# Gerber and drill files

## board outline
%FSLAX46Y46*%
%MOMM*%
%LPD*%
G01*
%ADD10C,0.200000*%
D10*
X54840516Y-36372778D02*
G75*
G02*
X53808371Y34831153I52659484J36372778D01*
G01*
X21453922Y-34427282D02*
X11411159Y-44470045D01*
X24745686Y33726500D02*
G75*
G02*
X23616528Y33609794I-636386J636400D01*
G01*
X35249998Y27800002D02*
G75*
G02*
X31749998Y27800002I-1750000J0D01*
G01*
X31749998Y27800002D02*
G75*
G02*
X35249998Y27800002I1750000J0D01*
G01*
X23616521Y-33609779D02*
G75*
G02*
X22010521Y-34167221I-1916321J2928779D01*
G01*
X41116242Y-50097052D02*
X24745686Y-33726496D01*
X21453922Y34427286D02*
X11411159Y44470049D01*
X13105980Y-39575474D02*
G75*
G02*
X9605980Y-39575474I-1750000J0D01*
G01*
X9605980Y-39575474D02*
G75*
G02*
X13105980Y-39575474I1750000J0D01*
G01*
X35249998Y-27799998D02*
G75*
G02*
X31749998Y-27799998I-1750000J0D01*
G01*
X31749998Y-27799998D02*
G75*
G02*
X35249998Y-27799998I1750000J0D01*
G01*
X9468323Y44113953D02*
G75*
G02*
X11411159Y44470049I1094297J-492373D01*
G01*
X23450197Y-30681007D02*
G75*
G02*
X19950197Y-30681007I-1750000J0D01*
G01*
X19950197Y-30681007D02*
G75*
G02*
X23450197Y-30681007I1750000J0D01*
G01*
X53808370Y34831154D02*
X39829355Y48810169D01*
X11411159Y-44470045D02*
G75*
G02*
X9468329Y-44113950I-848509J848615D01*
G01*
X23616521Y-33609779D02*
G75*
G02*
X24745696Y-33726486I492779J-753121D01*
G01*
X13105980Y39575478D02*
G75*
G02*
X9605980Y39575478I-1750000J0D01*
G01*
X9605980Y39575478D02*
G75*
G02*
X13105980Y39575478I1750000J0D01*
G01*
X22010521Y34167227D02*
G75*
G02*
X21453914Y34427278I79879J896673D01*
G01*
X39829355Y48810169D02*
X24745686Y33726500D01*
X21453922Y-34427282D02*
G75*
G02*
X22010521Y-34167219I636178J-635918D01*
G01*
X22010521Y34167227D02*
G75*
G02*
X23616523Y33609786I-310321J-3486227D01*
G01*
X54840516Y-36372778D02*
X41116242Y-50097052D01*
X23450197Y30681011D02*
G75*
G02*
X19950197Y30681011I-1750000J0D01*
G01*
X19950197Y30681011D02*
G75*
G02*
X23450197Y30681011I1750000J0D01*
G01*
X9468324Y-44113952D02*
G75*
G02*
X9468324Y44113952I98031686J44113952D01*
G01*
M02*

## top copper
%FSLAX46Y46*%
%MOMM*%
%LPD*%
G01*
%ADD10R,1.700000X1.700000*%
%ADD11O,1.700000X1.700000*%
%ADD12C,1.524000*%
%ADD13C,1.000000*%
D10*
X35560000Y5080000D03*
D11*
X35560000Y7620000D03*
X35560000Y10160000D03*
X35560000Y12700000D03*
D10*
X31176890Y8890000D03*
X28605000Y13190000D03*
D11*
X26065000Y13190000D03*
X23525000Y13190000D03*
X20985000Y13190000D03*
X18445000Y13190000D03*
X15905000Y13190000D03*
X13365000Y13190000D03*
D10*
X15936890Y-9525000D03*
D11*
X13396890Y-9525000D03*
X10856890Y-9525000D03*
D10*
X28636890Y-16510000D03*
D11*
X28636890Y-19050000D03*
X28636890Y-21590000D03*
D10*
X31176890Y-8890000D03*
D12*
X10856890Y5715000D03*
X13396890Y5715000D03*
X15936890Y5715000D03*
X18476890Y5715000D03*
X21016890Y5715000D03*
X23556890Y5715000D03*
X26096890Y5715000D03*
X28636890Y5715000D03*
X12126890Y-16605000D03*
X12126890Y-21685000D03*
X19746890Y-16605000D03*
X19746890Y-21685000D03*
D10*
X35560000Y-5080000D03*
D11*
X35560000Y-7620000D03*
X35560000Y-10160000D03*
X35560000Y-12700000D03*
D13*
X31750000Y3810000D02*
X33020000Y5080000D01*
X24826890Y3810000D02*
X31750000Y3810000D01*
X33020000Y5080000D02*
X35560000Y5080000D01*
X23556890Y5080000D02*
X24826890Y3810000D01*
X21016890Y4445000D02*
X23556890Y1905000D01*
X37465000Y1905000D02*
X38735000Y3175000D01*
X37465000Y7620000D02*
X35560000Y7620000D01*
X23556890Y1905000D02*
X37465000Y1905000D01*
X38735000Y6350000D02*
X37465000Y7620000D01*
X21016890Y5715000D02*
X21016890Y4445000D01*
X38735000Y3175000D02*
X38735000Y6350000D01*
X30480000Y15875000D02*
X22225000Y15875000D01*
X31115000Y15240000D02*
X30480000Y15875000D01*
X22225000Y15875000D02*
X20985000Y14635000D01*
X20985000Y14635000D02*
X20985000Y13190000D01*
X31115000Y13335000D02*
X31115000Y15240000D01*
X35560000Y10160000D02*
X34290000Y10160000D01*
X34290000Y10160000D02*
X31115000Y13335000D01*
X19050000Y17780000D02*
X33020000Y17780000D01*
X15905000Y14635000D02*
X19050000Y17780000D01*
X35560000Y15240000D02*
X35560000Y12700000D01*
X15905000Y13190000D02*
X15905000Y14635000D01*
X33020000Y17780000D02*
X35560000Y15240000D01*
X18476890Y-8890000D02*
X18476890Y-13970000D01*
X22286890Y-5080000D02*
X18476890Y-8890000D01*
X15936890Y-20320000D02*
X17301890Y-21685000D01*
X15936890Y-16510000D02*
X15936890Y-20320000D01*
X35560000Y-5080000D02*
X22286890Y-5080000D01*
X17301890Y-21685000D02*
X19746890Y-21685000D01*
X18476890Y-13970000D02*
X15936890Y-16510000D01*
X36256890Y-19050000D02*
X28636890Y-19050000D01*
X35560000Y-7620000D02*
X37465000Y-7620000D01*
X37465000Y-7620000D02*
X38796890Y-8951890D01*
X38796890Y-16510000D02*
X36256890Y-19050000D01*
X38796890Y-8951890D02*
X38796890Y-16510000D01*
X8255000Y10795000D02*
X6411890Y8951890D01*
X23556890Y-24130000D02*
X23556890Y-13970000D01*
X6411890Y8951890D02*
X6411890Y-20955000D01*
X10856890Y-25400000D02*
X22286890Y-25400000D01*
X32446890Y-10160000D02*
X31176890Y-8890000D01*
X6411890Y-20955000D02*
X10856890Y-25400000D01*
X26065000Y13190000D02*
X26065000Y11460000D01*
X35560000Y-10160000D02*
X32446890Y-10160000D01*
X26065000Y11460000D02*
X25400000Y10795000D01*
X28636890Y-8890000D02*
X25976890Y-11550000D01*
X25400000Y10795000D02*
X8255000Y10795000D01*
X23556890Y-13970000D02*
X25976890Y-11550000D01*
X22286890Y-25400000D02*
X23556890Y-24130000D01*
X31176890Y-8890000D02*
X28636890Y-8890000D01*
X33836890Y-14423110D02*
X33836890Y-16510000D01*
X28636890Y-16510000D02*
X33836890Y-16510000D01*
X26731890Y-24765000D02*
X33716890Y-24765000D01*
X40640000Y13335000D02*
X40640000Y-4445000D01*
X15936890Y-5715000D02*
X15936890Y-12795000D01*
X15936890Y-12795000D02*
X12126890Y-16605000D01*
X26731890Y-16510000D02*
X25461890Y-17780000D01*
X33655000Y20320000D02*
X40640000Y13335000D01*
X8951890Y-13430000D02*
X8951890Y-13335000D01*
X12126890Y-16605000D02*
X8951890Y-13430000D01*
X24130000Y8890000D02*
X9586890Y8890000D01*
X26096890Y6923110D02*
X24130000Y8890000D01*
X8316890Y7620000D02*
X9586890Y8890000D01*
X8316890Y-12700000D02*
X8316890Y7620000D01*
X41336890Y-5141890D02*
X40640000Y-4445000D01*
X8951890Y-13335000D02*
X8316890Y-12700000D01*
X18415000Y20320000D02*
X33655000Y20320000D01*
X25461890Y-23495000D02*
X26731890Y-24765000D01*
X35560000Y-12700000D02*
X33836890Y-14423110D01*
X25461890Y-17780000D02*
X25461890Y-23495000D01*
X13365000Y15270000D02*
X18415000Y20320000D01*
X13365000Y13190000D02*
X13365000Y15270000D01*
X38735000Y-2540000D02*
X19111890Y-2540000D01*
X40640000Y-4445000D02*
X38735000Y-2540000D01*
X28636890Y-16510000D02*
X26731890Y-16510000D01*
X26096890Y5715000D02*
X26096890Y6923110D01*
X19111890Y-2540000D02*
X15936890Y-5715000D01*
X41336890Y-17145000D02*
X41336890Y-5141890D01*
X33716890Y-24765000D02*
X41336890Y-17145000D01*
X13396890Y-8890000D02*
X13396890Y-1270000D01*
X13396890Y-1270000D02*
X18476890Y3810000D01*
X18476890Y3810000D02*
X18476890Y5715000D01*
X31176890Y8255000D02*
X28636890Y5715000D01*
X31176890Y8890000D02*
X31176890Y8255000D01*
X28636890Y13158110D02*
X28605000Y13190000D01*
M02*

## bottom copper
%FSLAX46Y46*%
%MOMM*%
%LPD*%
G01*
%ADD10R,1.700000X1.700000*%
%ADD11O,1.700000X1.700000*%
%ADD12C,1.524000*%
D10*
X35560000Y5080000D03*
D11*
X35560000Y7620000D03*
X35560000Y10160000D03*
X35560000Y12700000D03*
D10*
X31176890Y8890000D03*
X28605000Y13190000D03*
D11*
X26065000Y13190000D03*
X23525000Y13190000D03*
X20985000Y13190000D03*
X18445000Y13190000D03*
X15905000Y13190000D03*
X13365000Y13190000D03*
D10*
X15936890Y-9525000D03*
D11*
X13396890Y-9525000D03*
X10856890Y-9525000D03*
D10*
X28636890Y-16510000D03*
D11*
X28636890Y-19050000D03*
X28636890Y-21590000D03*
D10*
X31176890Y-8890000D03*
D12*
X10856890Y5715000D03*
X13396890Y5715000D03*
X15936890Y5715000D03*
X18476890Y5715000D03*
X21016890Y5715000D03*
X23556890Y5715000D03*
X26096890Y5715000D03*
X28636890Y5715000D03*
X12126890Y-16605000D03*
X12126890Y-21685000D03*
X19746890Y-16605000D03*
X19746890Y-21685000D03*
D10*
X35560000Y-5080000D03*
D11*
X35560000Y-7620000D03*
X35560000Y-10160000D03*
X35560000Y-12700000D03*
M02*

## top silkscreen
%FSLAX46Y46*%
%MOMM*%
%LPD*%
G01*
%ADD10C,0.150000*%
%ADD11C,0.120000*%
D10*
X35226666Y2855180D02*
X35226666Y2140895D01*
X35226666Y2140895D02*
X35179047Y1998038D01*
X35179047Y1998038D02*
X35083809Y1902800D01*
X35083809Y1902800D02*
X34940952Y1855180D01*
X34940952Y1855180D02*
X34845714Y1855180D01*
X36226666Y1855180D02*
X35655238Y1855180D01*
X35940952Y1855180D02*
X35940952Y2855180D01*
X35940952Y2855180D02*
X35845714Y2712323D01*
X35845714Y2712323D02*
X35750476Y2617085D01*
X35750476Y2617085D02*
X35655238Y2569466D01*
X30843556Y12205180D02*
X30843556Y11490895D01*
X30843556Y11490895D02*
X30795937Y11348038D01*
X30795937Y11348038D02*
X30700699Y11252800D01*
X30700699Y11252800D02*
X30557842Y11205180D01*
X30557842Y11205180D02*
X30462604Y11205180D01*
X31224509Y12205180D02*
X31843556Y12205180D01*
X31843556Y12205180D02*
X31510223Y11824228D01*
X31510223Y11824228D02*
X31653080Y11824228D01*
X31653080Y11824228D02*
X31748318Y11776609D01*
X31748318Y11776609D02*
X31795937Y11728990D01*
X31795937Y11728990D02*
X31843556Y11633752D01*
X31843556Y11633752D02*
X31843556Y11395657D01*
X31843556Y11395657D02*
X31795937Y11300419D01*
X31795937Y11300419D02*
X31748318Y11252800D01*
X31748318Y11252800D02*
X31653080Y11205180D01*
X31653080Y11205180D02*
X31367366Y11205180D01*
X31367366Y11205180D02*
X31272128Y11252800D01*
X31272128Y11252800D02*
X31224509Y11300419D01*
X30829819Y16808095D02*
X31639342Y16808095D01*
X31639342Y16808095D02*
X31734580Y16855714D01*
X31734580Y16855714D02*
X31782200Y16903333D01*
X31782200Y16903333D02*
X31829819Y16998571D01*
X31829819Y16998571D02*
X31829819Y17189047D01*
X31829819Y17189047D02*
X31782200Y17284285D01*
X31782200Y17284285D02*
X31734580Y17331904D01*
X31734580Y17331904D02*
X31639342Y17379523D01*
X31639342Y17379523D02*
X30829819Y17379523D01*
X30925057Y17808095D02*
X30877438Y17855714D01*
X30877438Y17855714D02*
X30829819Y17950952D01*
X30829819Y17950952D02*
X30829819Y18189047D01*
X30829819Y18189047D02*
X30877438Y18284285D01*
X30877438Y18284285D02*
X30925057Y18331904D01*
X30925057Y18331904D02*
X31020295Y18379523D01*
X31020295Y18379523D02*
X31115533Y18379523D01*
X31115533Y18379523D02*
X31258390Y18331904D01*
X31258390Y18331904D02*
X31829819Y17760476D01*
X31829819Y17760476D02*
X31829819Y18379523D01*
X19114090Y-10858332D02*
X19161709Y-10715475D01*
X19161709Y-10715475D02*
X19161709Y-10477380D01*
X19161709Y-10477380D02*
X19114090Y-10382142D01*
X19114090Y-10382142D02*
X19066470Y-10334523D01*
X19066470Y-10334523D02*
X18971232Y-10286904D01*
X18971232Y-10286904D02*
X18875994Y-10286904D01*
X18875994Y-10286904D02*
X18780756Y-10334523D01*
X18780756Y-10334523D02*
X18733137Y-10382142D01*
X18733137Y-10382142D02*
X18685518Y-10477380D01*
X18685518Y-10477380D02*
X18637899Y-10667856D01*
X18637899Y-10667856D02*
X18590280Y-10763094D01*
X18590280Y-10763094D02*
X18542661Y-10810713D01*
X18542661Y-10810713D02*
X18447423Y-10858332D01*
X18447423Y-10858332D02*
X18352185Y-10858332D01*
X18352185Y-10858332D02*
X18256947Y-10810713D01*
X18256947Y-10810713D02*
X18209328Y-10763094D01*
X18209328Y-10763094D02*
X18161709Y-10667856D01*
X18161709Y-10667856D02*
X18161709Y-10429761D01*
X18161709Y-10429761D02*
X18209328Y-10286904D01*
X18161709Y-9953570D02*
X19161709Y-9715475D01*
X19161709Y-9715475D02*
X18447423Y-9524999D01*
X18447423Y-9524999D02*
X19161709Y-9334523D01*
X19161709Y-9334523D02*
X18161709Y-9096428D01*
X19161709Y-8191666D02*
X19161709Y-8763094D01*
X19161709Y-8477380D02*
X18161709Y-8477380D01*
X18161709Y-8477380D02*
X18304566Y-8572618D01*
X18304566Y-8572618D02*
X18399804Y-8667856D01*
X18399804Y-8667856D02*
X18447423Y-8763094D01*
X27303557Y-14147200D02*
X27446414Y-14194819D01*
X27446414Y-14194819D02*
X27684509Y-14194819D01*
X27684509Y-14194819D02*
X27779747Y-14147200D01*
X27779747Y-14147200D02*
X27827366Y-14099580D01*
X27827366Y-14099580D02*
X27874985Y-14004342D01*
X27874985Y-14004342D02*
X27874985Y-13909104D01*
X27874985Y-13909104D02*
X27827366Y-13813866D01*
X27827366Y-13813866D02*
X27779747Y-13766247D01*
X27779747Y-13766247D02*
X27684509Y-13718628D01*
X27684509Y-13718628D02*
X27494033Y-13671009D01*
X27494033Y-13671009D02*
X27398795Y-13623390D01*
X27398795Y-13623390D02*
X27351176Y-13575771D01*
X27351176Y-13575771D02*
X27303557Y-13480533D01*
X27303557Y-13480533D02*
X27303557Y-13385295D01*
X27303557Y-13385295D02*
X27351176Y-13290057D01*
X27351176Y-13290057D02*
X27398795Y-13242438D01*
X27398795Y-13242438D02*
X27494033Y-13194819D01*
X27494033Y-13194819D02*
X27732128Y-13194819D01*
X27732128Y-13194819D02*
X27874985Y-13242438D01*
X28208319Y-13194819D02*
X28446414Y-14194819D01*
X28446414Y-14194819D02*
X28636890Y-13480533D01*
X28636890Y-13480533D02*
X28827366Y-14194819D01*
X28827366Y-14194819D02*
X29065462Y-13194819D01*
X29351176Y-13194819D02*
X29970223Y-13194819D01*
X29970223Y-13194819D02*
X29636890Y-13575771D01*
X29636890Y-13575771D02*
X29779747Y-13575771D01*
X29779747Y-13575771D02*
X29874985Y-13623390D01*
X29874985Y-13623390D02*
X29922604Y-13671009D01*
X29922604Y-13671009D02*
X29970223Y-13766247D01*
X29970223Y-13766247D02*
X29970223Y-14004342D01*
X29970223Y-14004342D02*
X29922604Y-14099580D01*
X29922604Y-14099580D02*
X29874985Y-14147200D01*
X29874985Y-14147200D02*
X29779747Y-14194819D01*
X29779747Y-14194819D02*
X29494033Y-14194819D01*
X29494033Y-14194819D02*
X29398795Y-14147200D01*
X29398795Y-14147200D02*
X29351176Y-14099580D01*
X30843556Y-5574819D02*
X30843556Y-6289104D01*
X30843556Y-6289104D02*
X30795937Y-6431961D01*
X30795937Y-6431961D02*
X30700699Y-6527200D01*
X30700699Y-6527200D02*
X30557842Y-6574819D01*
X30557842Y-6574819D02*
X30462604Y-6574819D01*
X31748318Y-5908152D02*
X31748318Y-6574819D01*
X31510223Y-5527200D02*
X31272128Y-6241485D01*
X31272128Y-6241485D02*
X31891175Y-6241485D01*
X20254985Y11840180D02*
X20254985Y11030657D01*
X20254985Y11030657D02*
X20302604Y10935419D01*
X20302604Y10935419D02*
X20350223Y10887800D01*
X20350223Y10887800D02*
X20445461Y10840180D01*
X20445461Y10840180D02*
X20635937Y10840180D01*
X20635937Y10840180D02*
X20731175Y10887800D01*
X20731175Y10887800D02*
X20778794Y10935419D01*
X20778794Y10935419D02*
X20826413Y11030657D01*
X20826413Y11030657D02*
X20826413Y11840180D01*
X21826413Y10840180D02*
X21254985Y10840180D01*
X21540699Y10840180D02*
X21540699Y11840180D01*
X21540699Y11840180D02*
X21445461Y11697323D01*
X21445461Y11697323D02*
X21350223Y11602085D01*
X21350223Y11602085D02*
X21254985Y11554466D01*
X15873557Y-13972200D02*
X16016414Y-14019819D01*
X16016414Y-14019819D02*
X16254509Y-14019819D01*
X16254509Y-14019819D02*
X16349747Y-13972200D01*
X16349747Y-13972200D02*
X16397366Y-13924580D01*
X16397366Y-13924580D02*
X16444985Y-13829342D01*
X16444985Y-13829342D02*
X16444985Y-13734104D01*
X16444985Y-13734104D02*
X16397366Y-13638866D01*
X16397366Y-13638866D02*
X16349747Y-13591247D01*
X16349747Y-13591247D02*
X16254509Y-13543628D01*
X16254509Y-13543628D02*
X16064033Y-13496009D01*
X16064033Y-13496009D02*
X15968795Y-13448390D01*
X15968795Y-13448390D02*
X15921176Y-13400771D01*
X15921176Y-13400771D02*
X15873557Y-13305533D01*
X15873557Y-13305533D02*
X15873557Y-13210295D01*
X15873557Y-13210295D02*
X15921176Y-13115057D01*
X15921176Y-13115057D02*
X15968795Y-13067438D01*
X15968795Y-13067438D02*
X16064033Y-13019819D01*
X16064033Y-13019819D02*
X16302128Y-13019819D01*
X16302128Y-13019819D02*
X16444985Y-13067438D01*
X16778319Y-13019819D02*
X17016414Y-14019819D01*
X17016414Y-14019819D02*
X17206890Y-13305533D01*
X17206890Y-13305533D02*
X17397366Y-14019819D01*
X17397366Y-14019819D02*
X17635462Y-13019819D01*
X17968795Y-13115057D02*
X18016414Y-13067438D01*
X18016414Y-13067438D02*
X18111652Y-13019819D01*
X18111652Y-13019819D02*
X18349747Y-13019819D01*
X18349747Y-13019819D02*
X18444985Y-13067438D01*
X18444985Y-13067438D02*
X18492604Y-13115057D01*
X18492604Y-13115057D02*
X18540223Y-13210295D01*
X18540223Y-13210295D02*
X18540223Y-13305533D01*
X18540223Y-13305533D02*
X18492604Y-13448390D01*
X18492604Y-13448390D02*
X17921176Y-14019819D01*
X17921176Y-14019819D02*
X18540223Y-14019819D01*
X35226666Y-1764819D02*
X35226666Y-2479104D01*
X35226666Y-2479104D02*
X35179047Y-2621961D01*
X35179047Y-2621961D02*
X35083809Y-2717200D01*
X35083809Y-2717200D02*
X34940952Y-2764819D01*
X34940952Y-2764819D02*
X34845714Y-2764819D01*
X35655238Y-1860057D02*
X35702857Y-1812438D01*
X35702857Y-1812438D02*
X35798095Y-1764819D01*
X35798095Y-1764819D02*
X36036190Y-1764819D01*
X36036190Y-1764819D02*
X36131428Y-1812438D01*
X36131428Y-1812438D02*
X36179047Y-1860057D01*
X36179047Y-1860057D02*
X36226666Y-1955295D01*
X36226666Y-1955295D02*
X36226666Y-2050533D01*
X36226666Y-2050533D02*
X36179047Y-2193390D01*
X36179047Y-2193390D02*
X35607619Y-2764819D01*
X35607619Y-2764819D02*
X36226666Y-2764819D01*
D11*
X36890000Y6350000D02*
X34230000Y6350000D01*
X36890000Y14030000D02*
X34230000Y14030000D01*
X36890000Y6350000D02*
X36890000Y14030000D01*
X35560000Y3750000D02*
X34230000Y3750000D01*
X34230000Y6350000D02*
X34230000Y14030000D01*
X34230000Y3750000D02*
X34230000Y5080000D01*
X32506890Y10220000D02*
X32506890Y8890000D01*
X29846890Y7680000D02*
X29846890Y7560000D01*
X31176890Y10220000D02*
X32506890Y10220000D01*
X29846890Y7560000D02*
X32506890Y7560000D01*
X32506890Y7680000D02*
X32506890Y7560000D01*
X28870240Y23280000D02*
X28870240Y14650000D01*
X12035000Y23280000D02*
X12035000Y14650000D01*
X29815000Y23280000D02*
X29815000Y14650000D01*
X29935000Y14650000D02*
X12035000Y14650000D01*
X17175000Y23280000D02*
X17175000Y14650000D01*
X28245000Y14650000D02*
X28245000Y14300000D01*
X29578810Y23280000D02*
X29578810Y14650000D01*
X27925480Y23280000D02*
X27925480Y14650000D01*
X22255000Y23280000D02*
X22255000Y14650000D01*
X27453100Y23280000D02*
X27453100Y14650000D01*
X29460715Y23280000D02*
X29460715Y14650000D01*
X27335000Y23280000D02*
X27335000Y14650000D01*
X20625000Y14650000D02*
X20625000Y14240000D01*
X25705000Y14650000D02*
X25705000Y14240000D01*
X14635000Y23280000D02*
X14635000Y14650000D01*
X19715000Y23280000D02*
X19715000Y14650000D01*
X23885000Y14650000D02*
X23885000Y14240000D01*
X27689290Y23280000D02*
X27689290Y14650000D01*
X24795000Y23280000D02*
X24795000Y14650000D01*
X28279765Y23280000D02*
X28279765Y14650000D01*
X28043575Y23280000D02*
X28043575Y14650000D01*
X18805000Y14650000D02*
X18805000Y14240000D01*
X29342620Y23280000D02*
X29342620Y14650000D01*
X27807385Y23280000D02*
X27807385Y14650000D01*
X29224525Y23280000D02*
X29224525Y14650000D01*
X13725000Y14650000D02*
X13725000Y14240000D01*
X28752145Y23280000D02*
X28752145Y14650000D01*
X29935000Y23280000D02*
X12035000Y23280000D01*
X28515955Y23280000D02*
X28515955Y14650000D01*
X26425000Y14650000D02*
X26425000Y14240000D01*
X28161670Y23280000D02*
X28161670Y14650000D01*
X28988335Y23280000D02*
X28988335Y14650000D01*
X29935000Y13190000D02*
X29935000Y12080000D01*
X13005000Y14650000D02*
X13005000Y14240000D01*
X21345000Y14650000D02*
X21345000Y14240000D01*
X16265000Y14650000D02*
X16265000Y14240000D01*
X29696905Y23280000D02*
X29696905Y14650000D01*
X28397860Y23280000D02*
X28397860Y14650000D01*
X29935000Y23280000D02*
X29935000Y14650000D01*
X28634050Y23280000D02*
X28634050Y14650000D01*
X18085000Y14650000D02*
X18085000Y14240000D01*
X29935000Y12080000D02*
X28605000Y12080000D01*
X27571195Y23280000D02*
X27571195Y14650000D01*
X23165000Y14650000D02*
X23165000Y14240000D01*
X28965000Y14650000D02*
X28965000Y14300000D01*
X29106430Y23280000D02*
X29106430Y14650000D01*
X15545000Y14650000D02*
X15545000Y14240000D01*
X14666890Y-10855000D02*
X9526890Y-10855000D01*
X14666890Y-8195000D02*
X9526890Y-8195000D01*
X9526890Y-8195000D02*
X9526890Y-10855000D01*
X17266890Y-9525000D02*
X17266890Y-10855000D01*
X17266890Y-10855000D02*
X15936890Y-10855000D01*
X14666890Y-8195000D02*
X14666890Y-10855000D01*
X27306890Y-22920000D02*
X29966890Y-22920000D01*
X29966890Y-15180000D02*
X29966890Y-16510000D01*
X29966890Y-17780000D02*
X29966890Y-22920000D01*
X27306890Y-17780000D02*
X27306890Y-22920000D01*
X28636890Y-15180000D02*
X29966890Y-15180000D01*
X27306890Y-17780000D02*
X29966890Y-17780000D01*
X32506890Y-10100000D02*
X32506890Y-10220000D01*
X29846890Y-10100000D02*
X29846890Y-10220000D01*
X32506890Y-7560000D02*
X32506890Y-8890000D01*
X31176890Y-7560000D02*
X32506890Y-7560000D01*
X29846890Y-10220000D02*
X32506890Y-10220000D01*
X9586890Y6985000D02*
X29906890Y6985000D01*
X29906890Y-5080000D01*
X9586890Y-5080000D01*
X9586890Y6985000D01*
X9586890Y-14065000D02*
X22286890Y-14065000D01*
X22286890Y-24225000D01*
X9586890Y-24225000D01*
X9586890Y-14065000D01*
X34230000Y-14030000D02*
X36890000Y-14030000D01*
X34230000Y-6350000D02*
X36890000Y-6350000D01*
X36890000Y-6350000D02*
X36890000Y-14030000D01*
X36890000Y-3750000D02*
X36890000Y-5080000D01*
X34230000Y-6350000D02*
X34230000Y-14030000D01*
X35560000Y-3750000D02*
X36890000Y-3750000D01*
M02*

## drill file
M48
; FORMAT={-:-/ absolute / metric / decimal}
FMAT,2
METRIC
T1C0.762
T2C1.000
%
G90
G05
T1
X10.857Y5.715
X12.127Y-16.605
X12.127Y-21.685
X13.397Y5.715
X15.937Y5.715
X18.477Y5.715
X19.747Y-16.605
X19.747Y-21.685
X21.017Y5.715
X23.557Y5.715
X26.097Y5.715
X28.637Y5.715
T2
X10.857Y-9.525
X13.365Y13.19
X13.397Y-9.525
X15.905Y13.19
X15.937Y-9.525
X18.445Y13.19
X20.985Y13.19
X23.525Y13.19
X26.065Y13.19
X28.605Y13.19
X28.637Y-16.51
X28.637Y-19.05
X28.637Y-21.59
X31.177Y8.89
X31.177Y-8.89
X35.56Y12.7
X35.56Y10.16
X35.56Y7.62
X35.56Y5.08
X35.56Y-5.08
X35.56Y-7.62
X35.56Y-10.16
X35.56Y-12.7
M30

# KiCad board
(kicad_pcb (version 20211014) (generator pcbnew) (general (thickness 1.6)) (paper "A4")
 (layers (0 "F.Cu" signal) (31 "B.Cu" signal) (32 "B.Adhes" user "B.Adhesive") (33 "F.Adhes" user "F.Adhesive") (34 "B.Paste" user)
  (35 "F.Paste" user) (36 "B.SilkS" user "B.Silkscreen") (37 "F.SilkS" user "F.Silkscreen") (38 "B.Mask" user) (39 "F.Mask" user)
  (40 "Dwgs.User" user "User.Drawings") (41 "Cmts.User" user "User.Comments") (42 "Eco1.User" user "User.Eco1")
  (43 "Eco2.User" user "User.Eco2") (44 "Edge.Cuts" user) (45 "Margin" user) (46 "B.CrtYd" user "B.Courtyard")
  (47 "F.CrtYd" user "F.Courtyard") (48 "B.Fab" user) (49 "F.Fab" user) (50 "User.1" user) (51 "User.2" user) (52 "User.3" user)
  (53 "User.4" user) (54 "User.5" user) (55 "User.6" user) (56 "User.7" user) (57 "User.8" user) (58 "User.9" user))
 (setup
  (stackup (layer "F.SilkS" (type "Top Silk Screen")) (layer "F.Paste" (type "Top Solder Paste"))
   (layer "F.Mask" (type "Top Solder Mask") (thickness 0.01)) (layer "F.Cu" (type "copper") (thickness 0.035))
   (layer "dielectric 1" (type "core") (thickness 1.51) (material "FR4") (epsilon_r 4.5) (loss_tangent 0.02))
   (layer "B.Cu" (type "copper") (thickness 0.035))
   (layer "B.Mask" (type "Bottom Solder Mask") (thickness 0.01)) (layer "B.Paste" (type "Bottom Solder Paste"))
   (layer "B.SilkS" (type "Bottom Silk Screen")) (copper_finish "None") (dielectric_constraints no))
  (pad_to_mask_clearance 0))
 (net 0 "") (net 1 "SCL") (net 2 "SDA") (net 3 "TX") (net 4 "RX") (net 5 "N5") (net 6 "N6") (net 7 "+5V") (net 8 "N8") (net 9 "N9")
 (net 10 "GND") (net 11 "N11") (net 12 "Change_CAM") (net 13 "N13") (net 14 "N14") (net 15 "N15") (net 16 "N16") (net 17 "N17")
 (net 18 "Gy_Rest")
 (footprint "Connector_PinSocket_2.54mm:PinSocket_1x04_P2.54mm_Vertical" (layer "F.Cu") (at 35.56 -5.08 180)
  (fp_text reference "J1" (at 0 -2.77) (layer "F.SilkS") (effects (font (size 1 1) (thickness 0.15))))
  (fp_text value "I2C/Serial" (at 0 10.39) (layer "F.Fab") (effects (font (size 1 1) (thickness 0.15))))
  (fp_line (start -1.33 1.27) (end 1.33 1.27) (layer "F.SilkS") (width 0.12))
  (fp_line (start -1.33 8.95) (end 1.33 8.95) (layer "F.SilkS") (width 0.12))
  (fp_line (start -1.33 1.27) (end -1.33 8.95) (layer "F.SilkS") (width 0.12))
  (fp_line (start 0 -1.33) (end 1.33 -1.33) (layer "F.SilkS") (width 0.12))
  (fp_line (start 1.33 1.27) (end 1.33 8.95) (layer "F.SilkS") (width 0.12))
  (fp_line (start 1.33 -1.33) (end 1.33 0) (layer "F.SilkS") (width 0.12))
  (pad "1" thru_hole rect (at 0 0 180) (size 1.7 1.7) (drill 1) (layers *.Cu *.Mask) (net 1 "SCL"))
  (pad "2" thru_hole oval (at 0 2.54 180) (size 1.7 1.7) (drill 1) (layers *.Cu *.Mask) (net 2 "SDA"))
  (pad "3" thru_hole oval (at 0 5.08 180) (size 1.7 1.7) (drill 1) (layers *.Cu *.Mask) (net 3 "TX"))
  (pad "4" thru_hole oval (at 0 7.62 180) (size 1.7 1.7) (drill 1) (layers *.Cu *.Mask) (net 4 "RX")))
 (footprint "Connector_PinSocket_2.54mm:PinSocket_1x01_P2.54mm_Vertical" (layer "F.Cu") (at 31.17689 -8.89)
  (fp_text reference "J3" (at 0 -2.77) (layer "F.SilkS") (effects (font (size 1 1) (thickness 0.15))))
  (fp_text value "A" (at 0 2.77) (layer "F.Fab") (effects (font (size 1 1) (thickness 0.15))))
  (fp_line (start 1.33 -1.33) (end 1.33 0) (layer "F.SilkS") (width 0.12))
  (fp_line (start -1.33 1.21) (end -1.33 1.33) (layer "F.SilkS") (width 0.12))
  (fp_line (start 0 -1.33) (end 1.33 -1.33) (layer "F.SilkS") (width 0.12))
  (fp_line (start -1.33 1.33) (end 1.33 1.33) (layer "F.SilkS") (width 0.12))
  (fp_line (start 1.33 1.21) (end 1.33 1.33) (layer "F.SilkS") (width 0.12))
  (pad "1" thru_hole rect (at 0 0) (size 1.7 1.7) (drill 1) (layers *.Cu *.Mask) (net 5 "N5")))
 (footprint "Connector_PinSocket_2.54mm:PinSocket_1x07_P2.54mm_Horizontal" (layer "F.Cu") (at 28.605 -13.19 -90)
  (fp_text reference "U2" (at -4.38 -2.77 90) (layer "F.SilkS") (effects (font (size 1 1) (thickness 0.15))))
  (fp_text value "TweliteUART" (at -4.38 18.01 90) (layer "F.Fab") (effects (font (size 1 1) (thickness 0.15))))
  (fp_line (start -10.09 -0.26524) (end -1.46 -0.26524) (layer "F.SilkS") (width 0.12))
  (fp_line (start -10.09 16.57) (end -1.46 16.57) (layer "F.SilkS") (width 0.12))
  (fp_line (start -10.09 -1.21) (end -1.46 -1.21) (layer "F.SilkS") (width 0.12))
  (fp_line (start -1.46 -1.33) (end -1.46 16.57) (layer "F.SilkS") (width 0.12))
  (fp_line (start -10.09 11.43) (end -1.46 11.43) (layer "F.SilkS") (width 0.12))
  (fp_line (start -1.46 0.36) (end -1.11 0.36) (layer "F.SilkS") (width 0.12))
  (fp_line (start -10.09 -0.97381) (end -1.46 -0.97381) (layer "F.SilkS") (width 0.12))
  (fp_line (start -10.09 0.67952) (end -1.46 0.67952) (layer "F.SilkS") (width 0.12))
  (fp_line (start -10.09 6.35) (end -1.46 6.35) (layer "F.SilkS") (width 0.12))
  (fp_line (start -10.09 1.1519) (end -1.46 1.1519) (layer "F.SilkS") (width 0.12))
  (fp_line (start -10.09 -0.855715) (end -1.46 -0.855715) (layer "F.SilkS") (width 0.12))
  (fp_line (start -10.09 1.27) (end -1.46 1.27) (layer "F.SilkS") (width 0.12))
  (fp_line (start -1.46 7.98) (end -1.05 7.98) (layer "F.SilkS") (width 0.12))
  (fp_line (start -1.46 2.9) (end -1.05 2.9) (layer "F.SilkS") (width 0.12))
  (fp_line (start -10.09 13.97) (end -1.46 13.97) (layer "F.SilkS") (width 0.12))
  (fp_line (start -10.09 8.89) (end -1.46 8.89) (layer "F.SilkS") (width 0.12))
  (fp_line (start -1.46 4.72) (end -1.05 4.72) (layer "F.SilkS") (width 0.12))
  (fp_line (start -10.09 0.91571) (end -1.46 0.91571) (layer "F.SilkS") (width 0.12))
  (fp_line (start -10.09 3.81) (end -1.46 3.81) (layer "F.SilkS") (width 0.12))
  (fp_line (start -10.09 0.325235) (end -1.46 0.325235) (layer "F.SilkS") (width 0.12))
  (fp_line (start -10.09 0.561425) (end -1.46 0.561425) (layer "F.SilkS") (width 0.12))
  (fp_line (start -1.46 9.8) (end -1.05 9.8) (layer "F.SilkS") (width 0.12))
  (fp_line (start -10.09 -0.73762) (end -1.46 -0.73762) (layer "F.SilkS") (width 0.12))
  (fp_line (start -10.09 0.797615) (end -1.46 0.797615) (layer "F.SilkS") (width 0.12))
  (fp_line (start -10.09 -0.619525) (end -1.46 -0.619525) (layer "F.SilkS") (width 0.12))
  (fp_line (start -1.46 14.88) (end -1.05 14.88) (layer "F.SilkS") (width 0.12))
  (fp_line (start -10.09 -0.147145) (end -1.46 -0.147145) (layer "F.SilkS") (width 0.12))
  (fp_line (start -10.09 -1.33) (end -10.09 16.57) (layer "F.SilkS") (width 0.12))
  (fp_line (start -10.09 0.089045) (end -1.46 0.089045) (layer "F.SilkS") (width 0.12))
  (fp_line (start -1.46 2.18) (end -1.05 2.18) (layer "F.SilkS") (width 0.12))
  (fp_line (start -10.09 0.44333) (end -1.46 0.44333) (layer "F.SilkS") (width 0.12))
  (fp_line (start -10.09 -0.383335) (end -1.46 -0.383335) (layer "F.SilkS") (width 0.12))
  (fp_line (start 0 -1.33) (end 1.11 -1.33) (layer "F.SilkS") (width 0.12))
  (fp_line (start -1.46 15.6) (end -1.05 15.6) (layer "F.SilkS") (width 0.12))
  (fp_line (start -1.46 7.26) (end -1.05 7.26) (layer "F.SilkS") (width 0.12))
  (fp_line (start -1.46 12.34) (end -1.05 12.34) (layer "F.SilkS") (width 0.12))
  (fp_line (start -10.09 -1.091905) (end -1.46 -1.091905) (layer "F.SilkS") (width 0.12))
  (fp_line (start -10.09 0.20714) (end -1.46 0.20714) (layer "F.SilkS") (width 0.12))
  (fp_line (start -10.09 -1.33) (end -1.46 -1.33) (layer "F.SilkS") (width 0.12))
  (fp_line (start -10.09 -0.02905) (end -1.46 -0.02905) (layer "F.SilkS") (width 0.12))
  (fp_line (start -1.46 10.52) (end -1.05 10.52) (layer "F.SilkS") (width 0.12))
  (fp_line (start 1.11 -1.33) (end 1.11 0) (layer "F.SilkS") (width 0.12))
  (fp_line (start -10.09 1.033805) (end -1.46 1.033805) (layer "F.SilkS") (width 0.12))
  (fp_line (start -1.46 5.44) (end -1.05 5.44) (layer "F.SilkS") (width 0.12))
  (fp_line (start -1.46 -0.36) (end -1.11 -0.36) (layer "F.SilkS") (width 0.12))
  (fp_line (start -10.09 -0.50143) (end -1.46 -0.50143) (layer "F.SilkS") (width 0.12))
  (fp_line (start -1.46 13.06) (end -1.05 13.06) (layer "F.SilkS") (width 0.12))
  (pad "1" thru_hole rect (at 0 0 270) (size 1.7 1.7) (drill 1) (layers *.Cu *.Mask) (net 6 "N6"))
  (pad "2" thru_hole oval (at 0 2.54 270) (size 1.7 1.7) (drill 1) (layers *.Cu *.Mask) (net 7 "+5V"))
  (pad "3" thru_hole oval (at 0 5.08 270) (size 1.7 1.7) (drill 1) (layers *.Cu *.Mask) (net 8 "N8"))
  (pad "4" thru_hole oval (at 0 7.62 270) (size 1.7 1.7) (drill 1) (layers *.Cu *.Mask) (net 3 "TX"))
  (pad "5" thru_hole oval (at 0 10.16 270) (size 1.7 1.7) (drill 1) (layers *.Cu *.Mask) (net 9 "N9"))
  (pad "6" thru_hole oval (at 0 12.7 270) (size 1.7 1.7) (drill 1) (layers *.Cu *.Mask) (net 4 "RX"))
  (pad "7" thru_hole oval (at 0 15.24 270) (size 1.7 1.7) (drill 1) (layers *.Cu *.Mask) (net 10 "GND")))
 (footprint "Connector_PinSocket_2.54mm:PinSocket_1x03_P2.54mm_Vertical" (layer "F.Cu") (at 15.93689 9.525 -90)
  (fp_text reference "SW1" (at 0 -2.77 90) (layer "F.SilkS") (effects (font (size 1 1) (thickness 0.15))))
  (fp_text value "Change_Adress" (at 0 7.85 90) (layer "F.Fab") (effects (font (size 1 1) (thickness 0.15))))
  (fp_line (start 1.33 1.27) (end 1.33 6.41) (layer "F.SilkS") (width 0.12))
  (fp_line (start -1.33 1.27) (end -1.33 6.41) (layer "F.SilkS") (width 0.12))
  (fp_line (start -1.33 6.41) (end 1.33 6.41) (layer "F.SilkS") (width 0.12))
  (fp_line (start 0 -1.33) (end 1.33 -1.33) (layer "F.SilkS") (width 0.12))
  (fp_line (start 1.33 -1.33) (end 1.33 0) (layer "F.SilkS") (width 0.12))
  (fp_line (start -1.33 1.27) (end 1.33 1.27) (layer "F.SilkS") (width 0.12))
  (pad "1" thru_hole rect (at 0 0 270) (size 1.7 1.7) (drill 1) (layers *.Cu *.Mask) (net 10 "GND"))
  (pad "2" thru_hole oval (at 0 2.54 270) (size 1.7 1.7) (drill 1) (layers *.Cu *.Mask) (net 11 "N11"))
  (pad "3" thru_hole oval (at 0 5.08 270) (size 1.7 1.7) (drill 1) (layers *.Cu *.Mask)))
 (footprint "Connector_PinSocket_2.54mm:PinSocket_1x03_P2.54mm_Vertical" (layer "F.Cu") (at 28.63689 16.51)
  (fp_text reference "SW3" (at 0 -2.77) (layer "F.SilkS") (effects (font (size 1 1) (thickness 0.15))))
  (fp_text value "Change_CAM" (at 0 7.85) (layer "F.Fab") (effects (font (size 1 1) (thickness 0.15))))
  (fp_line (start -1.33 6.41) (end 1.33 6.41) (layer "F.SilkS") (width 0.12))
  (fp_line (start 1.33 -1.33) (end 1.33 0) (layer "F.SilkS") (width 0.12))
  (fp_line (start 1.33 1.27) (end 1.33 6.41) (layer "F.SilkS") (width 0.12))
  (fp_line (start -1.33 1.27) (end -1.33 6.41) (layer "F.SilkS") (width 0.12))
  (fp_line (start 0 -1.33) (end 1.33 -1.33) (layer "F.SilkS") (width 0.12))
  (fp_line (start -1.33 1.27) (end 1.33 1.27) (layer "F.SilkS") (width 0.12))
  (pad "1" thru_hole rect (at 0 0) (size 1.7 1.7) (drill 1) (layers *.Cu *.Mask) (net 10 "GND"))
  (pad "2" thru_hole oval (at 0 2.54) (size 1.7 1.7) (drill 1) (layers *.Cu *.Mask) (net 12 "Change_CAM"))
  (pad "3" thru_hole oval (at 0 5.08) (size 1.7 1.7) (drill 1) (layers *.Cu *.Mask)))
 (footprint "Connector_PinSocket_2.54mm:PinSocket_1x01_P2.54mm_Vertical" (layer "F.Cu") (at 31.17689 8.89)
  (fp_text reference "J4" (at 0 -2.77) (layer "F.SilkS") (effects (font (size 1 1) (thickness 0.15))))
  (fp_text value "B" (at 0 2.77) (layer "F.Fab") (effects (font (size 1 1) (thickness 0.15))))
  (fp_line (start 1.33 1.21) (end 1.33 1.33) (layer "F.SilkS") (width 0.12))
  (fp_line (start -1.33 1.21) (end -1.33 1.33) (layer "F.SilkS") (width 0.12))
  (fp_line (start 1.33 -1.33) (end 1.33 0) (layer "F.SilkS") (width 0.12))
  (fp_line (start 0 -1.33) (end 1.33 -1.33) (layer "F.SilkS") (width 0.12))
  (fp_line (start -1.33 1.33) (end 1.33 1.33) (layer "F.SilkS") (width 0.12))
  (pad "1" thru_hole rect (at 0 0) (size 1.7 1.7) (drill 1) (layers *.Cu *.Mask) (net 7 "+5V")))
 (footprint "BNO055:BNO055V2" (layer "F.Cu") (at 21.01689 -10.795)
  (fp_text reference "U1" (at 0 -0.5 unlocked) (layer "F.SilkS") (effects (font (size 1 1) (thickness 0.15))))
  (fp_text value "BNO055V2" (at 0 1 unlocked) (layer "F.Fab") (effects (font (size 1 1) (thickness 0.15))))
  (fp_rect (start -11.43 3.81) (end 8.89 15.875) (layer "F.SilkS") (width 0.12) (fill none))
  (pad "1" thru_hole circle (at -10.16 5.08) (size 1.524 1.524) (drill 0.762) (layers *.Cu *.Mask) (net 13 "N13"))
  (pad "2" thru_hole circle (at -7.62 5.08) (size 1.524 1.524) (drill 0.762) (layers *.Cu *.Mask) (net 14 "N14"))
  (pad "3" thru_hole circle (at -5.08 5.08) (size 1.524 1.524) (drill 0.762) (layers *.Cu *.Mask) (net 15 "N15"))
  (pad "4" thru_hole circle (at -2.54 5.08) (size 1.524 1.524) (drill 0.762) (layers *.Cu *.Mask) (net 11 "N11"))
  (pad "5" thru_hole circle (at 0 5.08) (size 1.524 1.524) (drill 0.762) (layers *.Cu *.Mask) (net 2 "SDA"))
  (pad "6" thru_hole circle (at 2.54 5.08) (size 1.524 1.524) (drill 0.762) (layers *.Cu *.Mask) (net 1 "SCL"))
  (pad "7" thru_hole circle (at 5.08 5.08) (size 1.524 1.524) (drill 0.762) (layers *.Cu *.Mask) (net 10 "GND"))
  (pad "8" thru_hole circle (at 7.62 5.08) (size 1.524 1.524) (drill 0.762) (layers *.Cu *.Mask) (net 5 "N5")))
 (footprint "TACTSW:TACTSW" (layer "F.Cu") (at 17.20689 14.065)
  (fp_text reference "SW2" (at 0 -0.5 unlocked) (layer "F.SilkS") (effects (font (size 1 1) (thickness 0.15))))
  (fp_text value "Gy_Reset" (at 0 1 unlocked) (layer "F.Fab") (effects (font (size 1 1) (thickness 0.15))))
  (fp_rect (start -7.62 0) (end 5.08 10.16) (layer "F.SilkS") (width 0.12) (fill none))
  (pad "1" thru_hole circle (at -5.08 2.54) (size 1.524 1.524) (drill 0.762) (layers *.Cu *.Mask) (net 10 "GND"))
  (pad "2" thru_hole circle (at -5.08 7.62) (size 1.524 1.524) (drill 0.762) (layers *.Cu *.Mask) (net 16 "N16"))
  (pad "3" thru_hole circle (at 2.54 2.54) (size 1.524 1.524) (drill 0.762) (layers *.Cu *.Mask) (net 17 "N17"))
  (pad "4" thru_hole circle (at 2.54 7.62) (size 1.524 1.524) (drill 0.762) (layers *.Cu *.Mask) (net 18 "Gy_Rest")))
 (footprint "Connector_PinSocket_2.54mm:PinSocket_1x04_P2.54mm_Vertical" (layer "F.Cu") (at 35.56 5.08)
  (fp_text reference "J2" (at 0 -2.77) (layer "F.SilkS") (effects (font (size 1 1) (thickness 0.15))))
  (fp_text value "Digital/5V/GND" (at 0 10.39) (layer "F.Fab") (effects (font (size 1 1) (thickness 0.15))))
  (fp_line (start -1.33 8.95) (end 1.33 8.95) (layer "F.SilkS") (width 0.12))
  (fp_line (start -1.33 1.27) (end 1.33 1.27) (layer "F.SilkS") (width 0.12))
  (fp_line (start 1.33 1.27) (end 1.33 8.95) (layer "F.SilkS") (width 0.12))
  (fp_line (start 1.33 -1.33) (end 1.33 0) (layer "F.SilkS") (width 0.12))
  (fp_line (start -1.33 1.27) (end -1.33 8.95) (layer "F.SilkS") (width 0.12))
  (fp_line (start 0 -1.33) (end 1.33 -1.33) (layer "F.SilkS") (width 0.12))
  (pad "1" thru_hole rect (at 0 0) (size 1.7 1.7) (drill 1) (layers *.Cu *.Mask) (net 18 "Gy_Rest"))
  (pad "2" thru_hole oval (at 0 2.54) (size 1.7 1.7) (drill 1) (layers *.Cu *.Mask) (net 12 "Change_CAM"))
  (pad "3" thru_hole oval (at 0 5.08) (size 1.7 1.7) (drill 1) (layers *.Cu *.Mask) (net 7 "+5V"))
  (pad "4" thru_hole oval (at 0 7.62) (size 1.7 1.7) (drill 1) (layers *.Cu *.Mask) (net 10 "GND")))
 (gr_arc (start 54.840516 36.372778) (mid 43.506721 0.927622) (end 53.80837 -34.831154) (layer "Edge.Cuts") (width 0.2))
 (gr_line (start 21.453922 34.427282) (end 11.411159 44.470045) (layer "Edge.Cuts") (width 0.2))
 (gr_arc (start 24.745686 -33.7265) (mid 24.201827 -33.467672) (end 23.616521 -33.609783) (layer "Edge.Cuts") (width 0.2))
 (gr_circle (center 33.499998 -27.800002) (end 31.749998 -27.800002) (layer "Edge.Cuts") (width 0.2) (fill none))
 (gr_arc (start 23.616521 33.609779) (mid 22.84788 33.987489) (end 22.010521 34.167223) (layer "Edge.Cuts") (width 0.2))
 (gr_line (start 41.116242 50.097052) (end 24.745686 33.726496) (layer "Edge.Cuts") (width 0.2))
 (gr_line (start 21.453922 -34.427286) (end 11.411159 -44.470049) (layer "Edge.Cuts") (width 0.2))
 (gr_circle (center 11.35598 39.575474) (end 9.60598 39.575474) (layer "Edge.Cuts") (width 0.2) (fill none))
 (gr_circle (center 33.499998 27.799998) (end 31.749998 27.799998) (layer "Edge.Cuts") (width 0.2) (fill none))
 (gr_arc (start 9.468323 -44.113953) (mid 10.346286 -44.801882) (end 11.411159 -44.470049) (layer "Edge.Cuts") (width 0.2))
 (gr_circle (center 21.700197 30.681007) (end 19.950197 30.681007) (layer "Edge.Cuts") (width 0.2) (fill none))
 (gr_line (start 53.80837 -34.831154) (end 39.829355 -48.810169) (layer "Edge.Cuts") (width 0.2))
 (gr_arc (start 11.411159 44.470045) (mid 10.3463 44.801819) (end 9.468324 44.113952) (layer "Edge.Cuts") (width 0.2))
 (gr_arc (start 23.616521 33.609779) (mid 24.201828 33.467658) (end 24.745686 33.726496) (layer "Edge.Cuts") (width 0.2))
 (gr_circle (center 11.35598 -39.575478) (end 9.60598 -39.575478) (layer "Edge.Cuts") (width 0.2) (fill none))
 (gr_arc (start 22.010521 -34.167227) (mid 21.709353 -34.248308) (end 21.453922 -34.427286) (layer "Edge.Cuts") (width 0.2))
 (gr_line (start 39.829355 -48.810169) (end 24.745686 -33.7265) (layer "Edge.Cuts") (width 0.2))
 (gr_arc (start 21.453922 34.427282) (mid 21.709335 34.248261) (end 22.010521 34.167223) (layer "Edge.Cuts") (width 0.2))
 (gr_arc (start 22.010521 -34.167227) (mid 22.84788 -33.987494) (end 23.616521 -33.609783) (layer "Edge.Cuts") (width 0.2))
 (gr_line (start 54.840516 36.372778) (end 41.116242 50.097052) (layer "Edge.Cuts") (width 0.2))
 (gr_circle (center 21.700197 -30.681011) (end 19.950197 -30.681011) (layer "Edge.Cuts") (width 0.2) (fill none))
 (gr_arc (start 9.468324 44.113952) (mid -0.000001 0) (end 9.468323 -44.113953) (layer "Edge.Cuts") (width 0.2))
 (segment (start 31.75 -3.81) (end 33.02 -5.08) (width 1) (layer "F.Cu") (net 1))
 (segment (start 24.82689 -3.81) (end 31.75 -3.81) (width 1) (layer "F.Cu") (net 1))
 (segment (start 33.02 -5.08) (end 35.56 -5.08) (width 1) (layer "F.Cu") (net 1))
 (segment (start 23.55689 -5.08) (end 24.82689 -3.81) (width 1) (layer "F.Cu") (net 1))
 (segment (start 21.01689 -4.445) (end 23.55689 -1.905) (width 1) (layer "F.Cu") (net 2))
 (segment (start 37.465 -1.905) (end 38.735 -3.175) (width 1) (layer "F.Cu") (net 2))
 (segment (start 37.465 -7.62) (end 35.56 -7.62) (width 1) (layer "F.Cu") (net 2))
 (segment (start 23.55689 -1.905) (end 37.465 -1.905) (width 1) (layer "F.Cu") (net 2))
 (segment (start 38.735 -6.35) (end 37.465 -7.62) (width 1) (layer "F.Cu") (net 2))
 (segment (start 21.01689 -5.715) (end 21.01689 -4.445) (width 1) (layer "F.Cu") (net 2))
 (segment (start 38.735 -3.175) (end 38.735 -6.35) (width 1) (layer "F.Cu") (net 2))
 (segment (start 30.48 -15.875) (end 22.225 -15.875) (width 1) (layer "F.Cu") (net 3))
 (segment (start 31.115 -15.24) (end 30.48 -15.875) (width 1) (layer "F.Cu") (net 3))
 (segment (start 22.225 -15.875) (end 20.985 -14.635) (width 1) (layer "F.Cu") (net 3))
 (segment (start 20.985 -14.635) (end 20.985 -13.19) (width 1) (layer "F.Cu") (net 3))
 (segment (start 31.115 -13.335) (end 31.115 -15.24) (width 1) (layer "F.Cu") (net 3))
 (segment (start 35.56 -10.16) (end 34.29 -10.16) (width 1) (layer "F.Cu") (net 3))
 (segment (start 34.29 -10.16) (end 31.115 -13.335) (width 1) (layer "F.Cu") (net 3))
 (segment (start 19.05 -17.78) (end 33.02 -17.78) (width 1) (layer "F.Cu") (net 4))
 (segment (start 15.905 -14.635) (end 19.05 -17.78) (width 1) (layer "F.Cu") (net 4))
 (segment (start 35.56 -15.24) (end 35.56 -12.7) (width 1) (layer "F.Cu") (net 4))
 (segment (start 15.905 -13.19) (end 15.905 -14.635) (width 1) (layer "F.Cu") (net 4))
 (segment (start 33.02 -17.78) (end 35.56 -15.24) (width 1) (layer "F.Cu") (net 4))
 (segment (start 18.47689 8.89) (end 18.47689 13.97) (width 1) (layer "F.Cu") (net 18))
 (segment (start 22.28689 5.08) (end 18.47689 8.89) (width 1) (layer "F.Cu") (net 18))
 (segment (start 15.93689 20.32) (end 17.30189 21.685) (width 1) (layer "F.Cu") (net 18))
 (segment (start 15.93689 16.51) (end 15.93689 20.32) (width 1) (layer "F.Cu") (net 18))
 (segment (start 35.56 5.08) (end 22.28689 5.08) (width 1) (layer "F.Cu") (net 18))
 (segment (start 17.30189 21.685) (end 19.74689 21.685) (width 1) (layer "F.Cu") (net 18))
 (segment (start 18.47689 13.97) (end 15.93689 16.51) (width 1) (layer "F.Cu") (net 18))
 (segment (start 36.25689 19.05) (end 28.63689 19.05) (width 1) (layer "F.Cu") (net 12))
 (segment (start 35.56 7.62) (end 37.465 7.62) (width 1) (layer "F.Cu") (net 12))
 (segment (start 37.465 7.62) (end 38.79689 8.95189) (width 1) (layer "F.Cu") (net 12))
 (segment (start 38.79689 16.51) (end 36.25689 19.05) (width 1) (layer "F.Cu") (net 12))
 (segment (start 38.79689 8.95189) (end 38.79689 16.51) (width 1) (layer "F.Cu") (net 12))
 (segment (start 8.255 -10.795) (end 6.41189 -8.95189) (width 1) (layer "F.Cu") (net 7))
 (segment (start 23.55689 24.13) (end 23.55689 13.97) (width 1) (layer "F.Cu") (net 7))
 (segment (start 6.41189 -8.95189) (end 6.41189 20.955) (width 1) (layer "F.Cu") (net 7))
 (segment (start 10.85689 25.4) (end 22.28689 25.4) (width 1) (layer "F.Cu") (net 7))
 (segment (start 32.44689 10.16) (end 31.17689 8.89) (width 1) (layer "F.Cu") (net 7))
 (segment (start 6.41189 20.955) (end 10.85689 25.4) (width 1) (layer "F.Cu") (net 7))
 (segment (start 26.065 -13.19) (end 26.065 -11.46) (width 1) (layer "F.Cu") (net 7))
 (segment (start 35.56 10.16) (end 32.44689 10.16) (width 1) (layer "F.Cu") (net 7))
 (segment (start 26.065 -11.46) (end 25.4 -10.795) (width 1) (layer "F.Cu") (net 7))
 (segment (start 28.63689 8.89) (end 25.97689 11.55) (width 1) (layer "F.Cu") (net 7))
 (segment (start 25.4 -10.795) (end 8.255 -10.795) (width 1) (layer "F.Cu") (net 7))
 (segment (start 23.55689 13.97) (end 25.97689 11.55) (width 1) (layer "F.Cu") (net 7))
 (segment (start 22.28689 25.4) (end 23.55689 24.13) (width 1) (layer "F.Cu") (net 7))
 (segment (start 31.17689 8.89) (end 28.63689 8.89) (width 1) (layer "F.Cu") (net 7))
 (segment (start 33.83689 14.42311) (end 33.83689 16.51) (width 1) (layer "F.Cu") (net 10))
 (segment (start 28.63689 16.51) (end 33.83689 16.51) (width 1) (layer "F.Cu") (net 10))
 (segment (start 26.73189 24.765) (end 33.71689 24.765) (width 1) (layer "F.Cu") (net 10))
 (segment (start 40.64 -13.335) (end 40.64 4.445) (width 1) (layer "F.Cu") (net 10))
 (segment (start 15.93689 5.715) (end 15.93689 12.795) (width 1) (layer "F.Cu") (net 10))
 (segment (start 15.93689 12.795) (end 12.12689 16.605) (width 1) (layer "F.Cu") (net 10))
 (segment (start 26.73189 16.51) (end 25.46189 17.78) (width 1) (layer "F.Cu") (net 10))
 (segment (start 33.655 -20.32) (end 40.64 -13.335) (width 1) (layer "F.Cu") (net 10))
 (segment (start 8.95189 13.43) (end 8.95189 13.335) (width 1) (layer "F.Cu") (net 10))
 (segment (start 12.12689 16.605) (end 8.95189 13.43) (width 1) (layer "F.Cu") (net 10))
 (segment (start 24.13 -8.89) (end 9.58689 -8.89) (width 1) (layer "F.Cu") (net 10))
 (segment (start 26.09689 -6.92311) (end 24.13 -8.89) (width 1) (layer "F.Cu") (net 10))
 (segment (start 8.31689 -7.62) (end 9.58689 -8.89) (width 1) (layer "F.Cu") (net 10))
 (segment (start 8.31689 12.7) (end 8.31689 -7.62) (width 1) (layer "F.Cu") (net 10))
 (segment (start 41.33689 5.14189) (end 40.64 4.445) (width 1) (layer "F.Cu") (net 10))
 (segment (start 8.95189 13.335) (end 8.31689 12.7) (width 1) (layer "F.Cu") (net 10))
 (segment (start 18.415 -20.32) (end 33.655 -20.32) (width 1) (layer "F.Cu") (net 10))
 (segment (start 25.46189 23.495) (end 26.73189 24.765) (width 1) (layer "F.Cu") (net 10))
 (segment (start 35.56 12.7) (end 33.83689 14.42311) (width 1) (layer "F.Cu") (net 10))
 (segment (start 25.46189 17.78) (end 25.46189 23.495) (width 1) (layer "F.Cu") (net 10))
 (segment (start 13.365 -15.27) (end 18.415 -20.32) (width 1) (layer "F.Cu") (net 10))
 (segment (start 13.365 -13.19) (end 13.365 -15.27) (width 1) (layer "F.Cu") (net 10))
 (segment (start 38.735 2.54) (end 19.11189 2.54) (width 1) (layer "F.Cu") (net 10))
 (segment (start 40.64 4.445) (end 38.735 2.54) (width 1) (layer "F.Cu") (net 10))
 (segment (start 28.63689 16.51) (end 26.73189 16.51) (width 1) (layer "F.Cu") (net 10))
 (segment (start 26.09689 -5.715) (end 26.09689 -6.92311) (width 1) (layer "F.Cu") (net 10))
 (segment (start 19.11189 2.54) (end 15.93689 5.715) (width 1) (layer "F.Cu") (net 10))
 (segment (start 41.33689 17.145) (end 41.33689 5.14189) (width 1) (layer "F.Cu") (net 10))
 (segment (start 33.71689 24.765) (end 41.33689 17.145) (width 1) (layer "F.Cu") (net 10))
 (segment (start 13.39689 8.89) (end 13.39689 1.27) (width 1) (layer "F.Cu") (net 11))
 (segment (start 13.39689 1.27) (end 18.47689 -3.81) (width 1) (layer "F.Cu") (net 11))
 (segment (start 18.47689 -3.81) (end 18.47689 -5.715) (width 1) (layer "F.Cu") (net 11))
 (segment (start 31.17689 -8.255) (end 28.63689 -5.715) (width 1) (layer "F.Cu") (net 5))
 (segment (start 31.17689 -8.89) (end 31.17689 -8.255) (width 1) (layer "F.Cu") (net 5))
 (segment (start 28.63689 -13.15811) (end 28.605 -13.19) (width 1) (layer "F.Cu") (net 6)))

